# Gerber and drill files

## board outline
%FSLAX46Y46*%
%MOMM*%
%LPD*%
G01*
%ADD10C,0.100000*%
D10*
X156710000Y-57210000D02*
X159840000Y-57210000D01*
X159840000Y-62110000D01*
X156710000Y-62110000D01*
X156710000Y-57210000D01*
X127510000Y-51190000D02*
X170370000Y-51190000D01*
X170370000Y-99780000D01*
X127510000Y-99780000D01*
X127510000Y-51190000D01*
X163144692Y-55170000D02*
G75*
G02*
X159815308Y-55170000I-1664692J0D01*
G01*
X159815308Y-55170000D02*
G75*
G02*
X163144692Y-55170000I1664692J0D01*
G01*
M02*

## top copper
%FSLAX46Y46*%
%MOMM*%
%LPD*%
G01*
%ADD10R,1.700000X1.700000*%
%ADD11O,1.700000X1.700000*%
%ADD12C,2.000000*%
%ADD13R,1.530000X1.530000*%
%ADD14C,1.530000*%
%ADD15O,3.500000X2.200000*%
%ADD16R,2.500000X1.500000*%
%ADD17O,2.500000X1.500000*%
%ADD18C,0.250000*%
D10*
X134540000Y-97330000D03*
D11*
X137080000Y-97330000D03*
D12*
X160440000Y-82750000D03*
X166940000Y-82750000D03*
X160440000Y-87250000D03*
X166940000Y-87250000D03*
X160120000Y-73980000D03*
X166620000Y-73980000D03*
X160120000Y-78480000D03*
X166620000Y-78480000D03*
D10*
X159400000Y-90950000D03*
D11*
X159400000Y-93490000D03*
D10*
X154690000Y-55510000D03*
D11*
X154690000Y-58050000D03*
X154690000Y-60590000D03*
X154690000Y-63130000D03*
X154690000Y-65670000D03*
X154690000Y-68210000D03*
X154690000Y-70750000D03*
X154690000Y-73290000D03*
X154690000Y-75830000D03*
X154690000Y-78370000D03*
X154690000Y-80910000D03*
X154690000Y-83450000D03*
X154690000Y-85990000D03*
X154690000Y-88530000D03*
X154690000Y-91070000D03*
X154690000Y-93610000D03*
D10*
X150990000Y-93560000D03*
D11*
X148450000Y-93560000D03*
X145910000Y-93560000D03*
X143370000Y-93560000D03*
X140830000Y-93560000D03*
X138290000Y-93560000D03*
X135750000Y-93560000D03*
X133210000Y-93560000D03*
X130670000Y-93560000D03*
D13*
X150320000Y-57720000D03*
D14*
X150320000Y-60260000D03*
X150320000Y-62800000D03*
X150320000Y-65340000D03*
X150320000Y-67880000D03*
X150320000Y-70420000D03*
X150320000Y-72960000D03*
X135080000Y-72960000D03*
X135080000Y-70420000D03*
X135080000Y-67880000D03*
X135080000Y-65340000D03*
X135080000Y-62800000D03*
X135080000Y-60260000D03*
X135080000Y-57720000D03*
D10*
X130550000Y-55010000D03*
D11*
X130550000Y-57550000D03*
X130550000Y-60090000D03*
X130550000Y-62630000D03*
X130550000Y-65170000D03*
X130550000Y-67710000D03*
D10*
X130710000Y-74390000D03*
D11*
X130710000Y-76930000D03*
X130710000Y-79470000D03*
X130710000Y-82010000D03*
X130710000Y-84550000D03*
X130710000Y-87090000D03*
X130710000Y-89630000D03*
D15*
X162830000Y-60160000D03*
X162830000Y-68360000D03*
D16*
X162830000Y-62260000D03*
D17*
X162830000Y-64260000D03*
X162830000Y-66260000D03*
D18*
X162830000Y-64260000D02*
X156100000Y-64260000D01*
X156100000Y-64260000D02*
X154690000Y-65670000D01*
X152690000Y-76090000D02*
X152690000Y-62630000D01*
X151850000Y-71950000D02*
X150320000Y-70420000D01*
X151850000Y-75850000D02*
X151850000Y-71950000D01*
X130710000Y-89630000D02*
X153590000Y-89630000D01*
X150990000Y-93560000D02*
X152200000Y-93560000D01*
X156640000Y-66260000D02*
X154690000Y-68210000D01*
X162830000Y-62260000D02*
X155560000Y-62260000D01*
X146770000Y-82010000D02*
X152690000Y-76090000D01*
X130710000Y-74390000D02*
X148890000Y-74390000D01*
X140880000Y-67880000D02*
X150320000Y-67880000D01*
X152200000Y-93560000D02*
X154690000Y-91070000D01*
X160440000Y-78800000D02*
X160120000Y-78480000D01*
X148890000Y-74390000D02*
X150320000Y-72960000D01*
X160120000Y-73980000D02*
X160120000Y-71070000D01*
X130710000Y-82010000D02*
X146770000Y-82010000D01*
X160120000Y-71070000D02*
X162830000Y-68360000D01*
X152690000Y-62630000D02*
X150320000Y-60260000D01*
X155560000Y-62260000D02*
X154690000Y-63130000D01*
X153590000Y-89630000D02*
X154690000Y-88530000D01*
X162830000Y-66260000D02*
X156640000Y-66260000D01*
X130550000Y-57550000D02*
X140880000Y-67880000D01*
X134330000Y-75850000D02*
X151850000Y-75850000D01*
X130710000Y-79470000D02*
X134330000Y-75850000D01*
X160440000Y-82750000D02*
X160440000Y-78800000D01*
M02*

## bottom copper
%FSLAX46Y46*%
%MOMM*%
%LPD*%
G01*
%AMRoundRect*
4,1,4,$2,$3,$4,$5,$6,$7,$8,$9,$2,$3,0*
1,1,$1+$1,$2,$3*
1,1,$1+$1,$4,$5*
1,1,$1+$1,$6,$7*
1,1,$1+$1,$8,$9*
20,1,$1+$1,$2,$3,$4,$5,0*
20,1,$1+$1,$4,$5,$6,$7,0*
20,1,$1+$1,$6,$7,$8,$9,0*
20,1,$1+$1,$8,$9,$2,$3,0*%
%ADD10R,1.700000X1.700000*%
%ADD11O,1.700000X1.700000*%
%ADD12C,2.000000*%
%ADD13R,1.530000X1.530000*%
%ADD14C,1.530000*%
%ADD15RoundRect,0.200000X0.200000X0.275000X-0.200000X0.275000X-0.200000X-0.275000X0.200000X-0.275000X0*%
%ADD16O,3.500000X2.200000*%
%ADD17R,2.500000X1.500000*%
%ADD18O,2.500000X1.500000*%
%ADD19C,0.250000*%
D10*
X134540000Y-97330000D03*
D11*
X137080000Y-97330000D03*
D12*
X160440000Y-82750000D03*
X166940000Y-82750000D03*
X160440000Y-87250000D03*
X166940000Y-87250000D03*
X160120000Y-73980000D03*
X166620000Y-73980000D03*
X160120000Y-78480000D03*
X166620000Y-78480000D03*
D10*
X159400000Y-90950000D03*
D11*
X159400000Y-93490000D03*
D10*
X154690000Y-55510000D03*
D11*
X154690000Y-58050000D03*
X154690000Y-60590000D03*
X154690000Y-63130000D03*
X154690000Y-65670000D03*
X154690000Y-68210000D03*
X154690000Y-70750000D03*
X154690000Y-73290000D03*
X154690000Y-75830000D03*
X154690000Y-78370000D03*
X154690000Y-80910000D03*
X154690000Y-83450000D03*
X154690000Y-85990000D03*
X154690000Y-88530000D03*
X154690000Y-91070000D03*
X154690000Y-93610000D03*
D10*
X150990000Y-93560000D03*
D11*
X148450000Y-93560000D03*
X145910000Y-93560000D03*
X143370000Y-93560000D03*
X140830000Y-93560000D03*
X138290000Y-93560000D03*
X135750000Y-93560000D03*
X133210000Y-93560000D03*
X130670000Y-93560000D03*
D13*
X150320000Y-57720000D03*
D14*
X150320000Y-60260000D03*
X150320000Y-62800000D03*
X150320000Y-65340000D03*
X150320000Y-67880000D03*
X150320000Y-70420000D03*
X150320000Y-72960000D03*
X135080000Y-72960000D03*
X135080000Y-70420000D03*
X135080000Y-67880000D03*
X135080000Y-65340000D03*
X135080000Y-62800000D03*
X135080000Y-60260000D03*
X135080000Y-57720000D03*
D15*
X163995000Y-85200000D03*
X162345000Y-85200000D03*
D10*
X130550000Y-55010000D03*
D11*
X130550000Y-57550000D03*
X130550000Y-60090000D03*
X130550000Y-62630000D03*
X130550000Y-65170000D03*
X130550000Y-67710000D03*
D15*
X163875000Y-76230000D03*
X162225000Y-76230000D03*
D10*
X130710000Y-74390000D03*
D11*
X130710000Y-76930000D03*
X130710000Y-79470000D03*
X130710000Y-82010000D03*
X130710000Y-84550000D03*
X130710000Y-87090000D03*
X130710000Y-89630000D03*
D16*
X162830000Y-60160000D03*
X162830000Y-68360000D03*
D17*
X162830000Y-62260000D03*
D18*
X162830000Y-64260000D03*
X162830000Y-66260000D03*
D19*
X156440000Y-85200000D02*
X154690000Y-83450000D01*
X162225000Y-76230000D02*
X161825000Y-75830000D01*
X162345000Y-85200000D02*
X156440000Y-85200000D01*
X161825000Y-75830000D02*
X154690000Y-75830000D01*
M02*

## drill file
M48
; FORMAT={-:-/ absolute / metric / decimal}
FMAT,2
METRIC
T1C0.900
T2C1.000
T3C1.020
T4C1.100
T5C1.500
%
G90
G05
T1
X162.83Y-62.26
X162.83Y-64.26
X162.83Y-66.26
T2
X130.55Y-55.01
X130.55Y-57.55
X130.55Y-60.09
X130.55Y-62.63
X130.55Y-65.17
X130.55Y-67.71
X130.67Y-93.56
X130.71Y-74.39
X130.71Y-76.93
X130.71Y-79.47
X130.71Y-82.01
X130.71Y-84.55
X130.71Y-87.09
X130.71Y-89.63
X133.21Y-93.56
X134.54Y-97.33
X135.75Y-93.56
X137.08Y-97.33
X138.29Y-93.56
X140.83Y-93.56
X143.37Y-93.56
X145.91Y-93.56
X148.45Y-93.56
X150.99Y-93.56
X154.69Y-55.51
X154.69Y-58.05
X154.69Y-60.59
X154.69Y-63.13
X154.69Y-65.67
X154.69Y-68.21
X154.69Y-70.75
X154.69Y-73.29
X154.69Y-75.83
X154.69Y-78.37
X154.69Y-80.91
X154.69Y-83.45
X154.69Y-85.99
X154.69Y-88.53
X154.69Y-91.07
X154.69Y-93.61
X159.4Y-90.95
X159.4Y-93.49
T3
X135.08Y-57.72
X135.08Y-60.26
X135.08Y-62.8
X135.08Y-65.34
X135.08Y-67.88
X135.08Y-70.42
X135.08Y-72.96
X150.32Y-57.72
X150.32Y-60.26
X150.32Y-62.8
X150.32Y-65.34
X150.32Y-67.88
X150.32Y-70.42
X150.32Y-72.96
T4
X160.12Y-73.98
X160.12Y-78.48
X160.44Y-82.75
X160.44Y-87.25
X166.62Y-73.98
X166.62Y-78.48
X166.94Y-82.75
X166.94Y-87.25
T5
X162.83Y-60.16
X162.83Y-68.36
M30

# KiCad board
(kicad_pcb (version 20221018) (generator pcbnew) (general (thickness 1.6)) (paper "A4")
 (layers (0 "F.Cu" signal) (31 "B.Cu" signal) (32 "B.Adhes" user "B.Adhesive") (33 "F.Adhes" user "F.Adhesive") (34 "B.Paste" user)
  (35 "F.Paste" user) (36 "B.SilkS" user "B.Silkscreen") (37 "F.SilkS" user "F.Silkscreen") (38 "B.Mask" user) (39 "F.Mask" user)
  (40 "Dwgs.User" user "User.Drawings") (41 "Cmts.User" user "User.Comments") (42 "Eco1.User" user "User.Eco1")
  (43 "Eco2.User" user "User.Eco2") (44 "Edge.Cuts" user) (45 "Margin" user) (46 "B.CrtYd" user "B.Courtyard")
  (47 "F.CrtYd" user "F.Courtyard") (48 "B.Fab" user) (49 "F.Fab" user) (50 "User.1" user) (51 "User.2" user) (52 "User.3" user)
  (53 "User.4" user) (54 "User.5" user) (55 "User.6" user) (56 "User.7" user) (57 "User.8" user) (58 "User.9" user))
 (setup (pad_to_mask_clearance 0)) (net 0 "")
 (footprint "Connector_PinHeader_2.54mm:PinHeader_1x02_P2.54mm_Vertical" (layer "F.Cu") (at 134.54 97.33 90)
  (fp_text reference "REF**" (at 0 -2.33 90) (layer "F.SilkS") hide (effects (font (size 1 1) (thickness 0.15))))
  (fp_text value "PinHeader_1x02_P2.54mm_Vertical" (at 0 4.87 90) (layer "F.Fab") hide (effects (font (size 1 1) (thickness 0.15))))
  (pad "1" thru_hole rect (at 0 0 90) (size 1.7 1.7) (drill 1) (layers "*.Cu" "*.Mask"))
  (pad "2" thru_hole oval (at 0 2.54 90) (size 1.7 1.7) (drill 1) (layers "*.Cu" "*.Mask")))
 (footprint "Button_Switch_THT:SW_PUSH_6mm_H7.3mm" (layer "F.Cu") (at 160.44 82.75)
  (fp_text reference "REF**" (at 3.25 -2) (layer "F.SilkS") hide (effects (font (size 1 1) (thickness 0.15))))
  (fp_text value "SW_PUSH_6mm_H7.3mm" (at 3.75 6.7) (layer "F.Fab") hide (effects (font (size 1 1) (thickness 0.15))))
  (pad "1" thru_hole circle (at 0 0 90) (size 2 2) (drill 1.1) (layers "*.Cu" "*.Mask"))
  (pad "1" thru_hole circle (at 6.5 0 90) (size 2 2) (drill 1.1) (layers "*.Cu" "*.Mask"))
  (pad "2" thru_hole circle (at 0 4.5 90) (size 2 2) (drill 1.1) (layers "*.Cu" "*.Mask"))
  (pad "2" thru_hole circle (at 6.5 4.5 90) (size 2 2) (drill 1.1) (layers "*.Cu" "*.Mask")))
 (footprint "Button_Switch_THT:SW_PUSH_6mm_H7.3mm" (layer "F.Cu") (at 160.12 73.98)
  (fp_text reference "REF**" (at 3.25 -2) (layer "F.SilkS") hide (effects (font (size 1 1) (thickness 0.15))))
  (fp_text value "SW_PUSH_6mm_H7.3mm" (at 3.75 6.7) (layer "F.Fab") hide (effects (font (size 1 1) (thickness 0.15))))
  (pad "1" thru_hole circle (at 0 0 90) (size 2 2) (drill 1.1) (layers "*.Cu" "*.Mask"))
  (pad "1" thru_hole circle (at 6.5 0 90) (size 2 2) (drill 1.1) (layers "*.Cu" "*.Mask"))
  (pad "2" thru_hole circle (at 0 4.5 90) (size 2 2) (drill 1.1) (layers "*.Cu" "*.Mask"))
  (pad "2" thru_hole circle (at 6.5 4.5 90) (size 2 2) (drill 1.1) (layers "*.Cu" "*.Mask")))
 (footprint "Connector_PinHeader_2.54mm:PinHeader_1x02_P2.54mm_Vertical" (layer "F.Cu") (at 159.4 90.95)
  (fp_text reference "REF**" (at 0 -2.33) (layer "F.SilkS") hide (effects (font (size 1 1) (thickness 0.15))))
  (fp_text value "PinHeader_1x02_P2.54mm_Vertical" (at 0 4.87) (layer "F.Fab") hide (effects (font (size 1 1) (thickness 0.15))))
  (pad "1" thru_hole rect (at 0 0) (size 1.7 1.7) (drill 1) (layers "*.Cu" "*.Mask"))
  (pad "2" thru_hole oval (at 0 2.54) (size 1.7 1.7) (drill 1) (layers "*.Cu" "*.Mask")))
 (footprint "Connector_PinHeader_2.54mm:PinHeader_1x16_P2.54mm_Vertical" (layer "B.Cu") (at 154.69 55.51 180)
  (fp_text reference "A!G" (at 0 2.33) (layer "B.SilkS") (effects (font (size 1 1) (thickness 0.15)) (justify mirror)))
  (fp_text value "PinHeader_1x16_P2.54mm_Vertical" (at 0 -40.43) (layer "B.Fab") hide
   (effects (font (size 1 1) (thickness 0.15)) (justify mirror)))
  (pad "1" thru_hole rect (at 0 0 180) (size 1.7 1.7) (drill 1) (layers "*.Cu" "*.Mask"))
  (pad "2" thru_hole oval (at 0 -2.54 180) (size 1.7 1.7) (drill 1) (layers "*.Cu" "*.Mask"))
  (pad "3" thru_hole oval (at 0 -5.08 180) (size 1.7 1.7) (drill 1) (layers "*.Cu" "*.Mask"))
  (pad "4" thru_hole oval (at 0 -7.62 180) (size 1.7 1.7) (drill 1) (layers "*.Cu" "*.Mask"))
  (pad "5" thru_hole oval (at 0 -10.16 180) (size 1.7 1.7) (drill 1) (layers "*.Cu" "*.Mask"))
  (pad "6" thru_hole oval (at 0 -12.7 180) (size 1.7 1.7) (drill 1) (layers "*.Cu" "*.Mask"))
  (pad "7" thru_hole oval (at 0 -15.24 180) (size 1.7 1.7) (drill 1) (layers "*.Cu" "*.Mask"))
  (pad "8" thru_hole oval (at 0 -17.78 180) (size 1.7 1.7) (drill 1) (layers "*.Cu" "*.Mask"))
  (pad "9" thru_hole oval (at 0 -20.32 180) (size 1.7 1.7) (drill 1) (layers "*.Cu" "*.Mask"))
  (pad "10" thru_hole oval (at 0 -22.86 180) (size 1.7 1.7) (drill 1) (layers "*.Cu" "*.Mask"))
  (pad "11" thru_hole oval (at 0 -25.4 180) (size 1.7 1.7) (drill 1) (layers "*.Cu" "*.Mask"))
  (pad "12" thru_hole oval (at 0 -27.94 180) (size 1.7 1.7) (drill 1) (layers "*.Cu" "*.Mask"))
  (pad "13" thru_hole oval (at 0 -30.48 180) (size 1.7 1.7) (drill 1) (layers "*.Cu" "*.Mask"))
  (pad "14" thru_hole oval (at 0 -33.02 180) (size 1.7 1.7) (drill 1) (layers "*.Cu" "*.Mask"))
  (pad "15" thru_hole oval (at 0 -35.56 180) (size 1.7 1.7) (drill 1) (layers "*.Cu" "*.Mask"))
  (pad "16" thru_hole oval (at 0 -38.1 180) (size 1.7 1.7) (drill 1) (layers "*.Cu" "*.Mask")))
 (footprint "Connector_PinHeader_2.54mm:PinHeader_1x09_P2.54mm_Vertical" (layer "B.Cu") (at 150.99 93.56 90)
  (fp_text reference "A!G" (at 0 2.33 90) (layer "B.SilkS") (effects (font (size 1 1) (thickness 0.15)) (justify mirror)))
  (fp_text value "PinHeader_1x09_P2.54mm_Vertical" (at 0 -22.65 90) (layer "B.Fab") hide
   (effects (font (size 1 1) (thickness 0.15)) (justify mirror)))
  (pad "1" thru_hole rect (at 0 0 90) (size 1.7 1.7) (drill 1) (layers "*.Cu" "*.Mask"))
  (pad "2" thru_hole oval (at 0 -2.54 90) (size 1.7 1.7) (drill 1) (layers "*.Cu" "*.Mask"))
  (pad "3" thru_hole oval (at 0 -5.08 90) (size 1.7 1.7) (drill 1) (layers "*.Cu" "*.Mask"))
  (pad "4" thru_hole oval (at 0 -7.62 90) (size 1.7 1.7) (drill 1) (layers "*.Cu" "*.Mask"))
  (pad "5" thru_hole oval (at 0 -10.16 90) (size 1.7 1.7) (drill 1) (layers "*.Cu" "*.Mask"))
  (pad "6" thru_hole oval (at 0 -12.7 90) (size 1.7 1.7) (drill 1) (layers "*.Cu" "*.Mask"))
  (pad "7" thru_hole oval (at 0 -15.24 90) (size 1.7 1.7) (drill 1) (layers "*.Cu" "*.Mask"))
  (pad "8" thru_hole oval (at 0 -17.78 90) (size 1.7 1.7) (drill 1) (layers "*.Cu" "*.Mask"))
  (pad "9" thru_hole oval (at 0 -20.32 90) (size 1.7 1.7) (drill 1) (layers "*.Cu" "*.Mask")))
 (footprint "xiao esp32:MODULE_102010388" (layer "B.Cu") (at 142.7 65.34 180)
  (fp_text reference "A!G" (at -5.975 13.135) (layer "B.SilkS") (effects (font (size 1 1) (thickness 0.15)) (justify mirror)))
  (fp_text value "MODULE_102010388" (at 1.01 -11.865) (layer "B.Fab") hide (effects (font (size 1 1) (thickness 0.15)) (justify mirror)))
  (pad "1" thru_hole rect (at -7.62 7.62 180) (size 1.53 1.53) (drill 1.02) (layers "*.Cu" "*.Mask") (solder_mask_margin 0.102))
  (pad "2" thru_hole circle (at -7.62 5.08 180) (size 1.53 1.53) (drill 1.02) (layers "*.Cu" "*.Mask") (solder_mask_margin 0.102))
  (pad "3" thru_hole circle (at -7.62 2.54 180) (size 1.53 1.53) (drill 1.02) (layers "*.Cu" "*.Mask") (solder_mask_margin 0.102))
  (pad "4" thru_hole circle (at -7.62 0 180) (size 1.53 1.53) (drill 1.02) (layers "*.Cu" "*.Mask") (solder_mask_margin 0.102))
  (pad "5" thru_hole circle (at -7.62 -2.54 180) (size 1.53 1.53) (drill 1.02) (layers "*.Cu" "*.Mask") (solder_mask_margin 0.102))
  (pad "6" thru_hole circle (at -7.62 -5.08 180) (size 1.53 1.53) (drill 1.02) (layers "*.Cu" "*.Mask") (solder_mask_margin 0.102))
  (pad "7" thru_hole circle (at -7.62 -7.62 180) (size 1.53 1.53) (drill 1.02) (layers "*.Cu" "*.Mask") (solder_mask_margin 0.102))
  (pad "8" thru_hole circle (at 7.62 -7.62 180) (size 1.53 1.53) (drill 1.02) (layers "*.Cu" "*.Mask") (solder_mask_margin 0.102))
  (pad "9" thru_hole circle (at 7.62 -5.08 180) (size 1.53 1.53) (drill 1.02) (layers "*.Cu" "*.Mask") (solder_mask_margin 0.102))
  (pad "10" thru_hole circle (at 7.62 -2.54 180) (size 1.53 1.53) (drill 1.02) (layers "*.Cu" "*.Mask") (solder_mask_margin 0.102))
  (pad "11" thru_hole circle (at 7.62 0 180) (size 1.53 1.53) (drill 1.02) (layers "*.Cu" "*.Mask") (solder_mask_margin 0.102))
  (pad "12" thru_hole circle (at 7.62 2.54 180) (size 1.53 1.53) (drill 1.02) (layers "*.Cu" "*.Mask") (solder_mask_margin 0.102))
  (pad "13" thru_hole circle (at 7.62 5.08 180) (size 1.53 1.53) (drill 1.02) (layers "*.Cu" "*.Mask") (solder_mask_margin 0.102))
  (pad "14" thru_hole circle (at 7.62 7.62 180) (size 1.53 1.53) (drill 1.02) (layers "*.Cu" "*.Mask") (solder_mask_margin 0.102)))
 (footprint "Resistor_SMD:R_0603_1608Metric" (layer "B.Cu") (at 163.17 85.2 180)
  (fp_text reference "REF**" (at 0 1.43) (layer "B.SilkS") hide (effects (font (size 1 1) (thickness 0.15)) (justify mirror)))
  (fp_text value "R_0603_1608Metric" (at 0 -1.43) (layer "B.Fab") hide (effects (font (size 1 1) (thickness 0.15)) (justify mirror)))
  (pad "1" smd roundrect (at -0.825 0 180) (size 0.8 0.95) (layers "B.Cu" "B.Paste" "B.Mask") (roundrect_rratio 0.25))
  (pad "2" smd roundrect (at 0.825 0 180) (size 0.8 0.95) (layers "B.Cu" "B.Paste" "B.Mask") (roundrect_rratio 0.25)))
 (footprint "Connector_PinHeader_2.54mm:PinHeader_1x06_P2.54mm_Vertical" (layer "B.Cu") (at 130.55 55.01 180)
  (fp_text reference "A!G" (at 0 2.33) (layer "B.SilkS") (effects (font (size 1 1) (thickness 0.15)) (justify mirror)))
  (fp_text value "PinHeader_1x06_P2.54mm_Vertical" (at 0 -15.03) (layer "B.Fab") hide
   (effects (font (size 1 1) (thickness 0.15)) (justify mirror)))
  (pad "1" thru_hole rect (at 0 0 180) (size 1.7 1.7) (drill 1) (layers "*.Cu" "*.Mask"))
  (pad "2" thru_hole oval (at 0 -2.54 180) (size 1.7 1.7) (drill 1) (layers "*.Cu" "*.Mask"))
  (pad "3" thru_hole oval (at 0 -5.08 180) (size 1.7 1.7) (drill 1) (layers "*.Cu" "*.Mask"))
  (pad "4" thru_hole oval (at 0 -7.62 180) (size 1.7 1.7) (drill 1) (layers "*.Cu" "*.Mask"))
  (pad "5" thru_hole oval (at 0 -10.16 180) (size 1.7 1.7) (drill 1) (layers "*.Cu" "*.Mask"))
  (pad "6" thru_hole oval (at 0 -12.7 180) (size 1.7 1.7) (drill 1) (layers "*.Cu" "*.Mask")))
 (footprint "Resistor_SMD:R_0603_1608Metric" (layer "B.Cu") (at 163.05 76.23 180)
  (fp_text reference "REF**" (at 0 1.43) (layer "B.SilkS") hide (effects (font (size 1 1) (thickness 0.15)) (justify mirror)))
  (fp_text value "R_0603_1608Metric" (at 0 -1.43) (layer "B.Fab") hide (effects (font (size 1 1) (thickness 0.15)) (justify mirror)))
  (pad "1" smd roundrect (at -0.825 0 180) (size 0.8 0.95) (layers "B.Cu" "B.Paste" "B.Mask") (roundrect_rratio 0.25))
  (pad "2" smd roundrect (at 0.825 0 180) (size 0.8 0.95) (layers "B.Cu" "B.Paste" "B.Mask") (roundrect_rratio 0.25)))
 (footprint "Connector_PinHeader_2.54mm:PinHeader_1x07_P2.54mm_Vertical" (layer "B.Cu") (at 130.71 74.39 180)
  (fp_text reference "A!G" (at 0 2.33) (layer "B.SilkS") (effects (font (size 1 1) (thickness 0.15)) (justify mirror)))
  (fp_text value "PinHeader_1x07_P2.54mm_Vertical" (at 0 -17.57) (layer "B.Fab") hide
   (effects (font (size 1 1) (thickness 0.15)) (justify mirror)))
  (pad "1" thru_hole rect (at 0 0 180) (size 1.7 1.7) (drill 1) (layers "*.Cu" "*.Mask"))
  (pad "2" thru_hole oval (at 0 -2.54 180) (size 1.7 1.7) (drill 1) (layers "*.Cu" "*.Mask"))
  (pad "3" thru_hole oval (at 0 -5.08 180) (size 1.7 1.7) (drill 1) (layers "*.Cu" "*.Mask"))
  (pad "4" thru_hole oval (at 0 -7.62 180) (size 1.7 1.7) (drill 1) (layers "*.Cu" "*.Mask"))
  (pad "5" thru_hole oval (at 0 -10.16 180) (size 1.7 1.7) (drill 1) (layers "*.Cu" "*.Mask"))
  (pad "6" thru_hole oval (at 0 -12.7 180) (size 1.7 1.7) (drill 1) (layers "*.Cu" "*.Mask"))
  (pad "7" thru_hole oval (at 0 -15.24 180) (size 1.7 1.7) (drill 1) (layers "*.Cu" "*.Mask")))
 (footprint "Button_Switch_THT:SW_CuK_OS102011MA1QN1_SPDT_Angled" (layer "B.Cu") (at 162.83 62.26 -90)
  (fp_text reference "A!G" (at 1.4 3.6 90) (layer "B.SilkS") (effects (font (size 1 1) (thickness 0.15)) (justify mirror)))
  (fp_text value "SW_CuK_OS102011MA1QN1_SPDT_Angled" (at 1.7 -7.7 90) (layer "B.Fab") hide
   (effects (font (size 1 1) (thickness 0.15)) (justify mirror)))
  (pad "" thru_hole oval (at -2.1 0 270) (size 2.2 3.5) (drill 1.5) (layers "*.Cu" "*.Mask"))
  (pad "" thru_hole oval (at 6.1 0 270) (size 2.2 3.5) (drill 1.5) (layers "*.Cu" "*.Mask"))
  (pad "1" thru_hole rect (at 0 0 270) (size 1.5 2.5) (drill 0.9) (layers "*.Cu" "*.Mask"))
  (pad "2" thru_hole oval (at 2 0 270) (size 1.5 2.5) (drill 0.9) (layers "*.Cu" "*.Mask"))
  (pad "3" thru_hole oval (at 4 0 270) (size 1.5 2.5) (drill 0.9) (layers "*.Cu" "*.Mask")))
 (gr_rect (start 156.71 57.21) (end 159.84 62.11) (stroke (width 0.1) (type default)) (fill none) (layer "Edge.Cuts"))
 (gr_rect (start 127.51 51.19) (end 170.37 99.78) (stroke (width 0.1) (type default)) (fill none) (layer "Edge.Cuts"))
 (gr_circle (center 161.48 55.17) (end 163.144692 55.17) (stroke (width 0.1) (type default)) (fill none) (layer "Edge.Cuts"))
 (segment (start 162.83 64.26) (end 156.1 64.26) (width 0.25) (layer "F.Cu") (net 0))
 (segment (start 156.1 64.26) (end 154.69 65.67) (width 0.25) (layer "F.Cu") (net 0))
 (segment (start 152.69 76.09) (end 152.69 62.63) (width 0.25) (layer "F.Cu") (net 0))
 (segment (start 151.85 71.95) (end 150.32 70.42) (width 0.25) (layer "F.Cu") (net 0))
 (segment (start 151.85 75.85) (end 151.85 71.95) (width 0.25) (layer "F.Cu") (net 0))
 (segment (start 130.71 89.63) (end 153.59 89.63) (width 0.25) (layer "F.Cu") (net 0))
 (segment (start 150.99 93.56) (end 152.2 93.56) (width 0.25) (layer "F.Cu") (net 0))
 (segment (start 156.64 66.26) (end 154.69 68.21) (width 0.25) (layer "F.Cu") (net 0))
 (segment (start 162.83 62.26) (end 155.56 62.26) (width 0.25) (layer "F.Cu") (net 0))
 (segment (start 146.77 82.01) (end 152.69 76.09) (width 0.25) (layer "F.Cu") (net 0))
 (segment (start 130.71 74.39) (end 148.89 74.39) (width 0.25) (layer "F.Cu") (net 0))
 (segment (start 140.88 67.88) (end 150.32 67.88) (width 0.25) (layer "F.Cu") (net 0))
 (segment (start 152.2 93.56) (end 154.69 91.07) (width 0.25) (layer "F.Cu") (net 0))
 (segment (start 160.44 78.8) (end 160.12 78.48) (width 0.25) (layer "F.Cu") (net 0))
 (segment (start 148.89 74.39) (end 150.32 72.96) (width 0.25) (layer "F.Cu") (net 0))
 (segment (start 160.12 73.98) (end 160.12 71.07) (width 0.25) (layer "F.Cu") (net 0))
 (segment (start 130.71 82.01) (end 146.77 82.01) (width 0.25) (layer "F.Cu") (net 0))
 (segment (start 160.12 71.07) (end 162.83 68.36) (width 0.25) (layer "F.Cu") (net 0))
 (segment (start 152.69 62.63) (end 150.32 60.26) (width 0.25) (layer "F.Cu") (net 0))
 (segment (start 155.56 62.26) (end 154.69 63.13) (width 0.25) (layer "F.Cu") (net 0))
 (segment (start 153.59 89.63) (end 154.69 88.53) (width 0.25) (layer "F.Cu") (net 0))
 (segment (start 162.83 66.26) (end 156.64 66.26) (width 0.25) (layer "F.Cu") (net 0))
 (segment (start 130.55 57.55) (end 140.88 67.88) (width 0.25) (layer "F.Cu") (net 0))
 (segment (start 134.33 75.85) (end 151.85 75.85) (width 0.25) (layer "F.Cu") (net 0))
 (segment (start 130.71 79.47) (end 134.33 75.85) (width 0.25) (layer "F.Cu") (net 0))
 (segment (start 160.44 82.75) (end 160.44 78.8) (width 0.25) (layer "F.Cu") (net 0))
 (segment (start 156.44 85.2) (end 154.69 83.45) (width 0.25) (layer "B.Cu") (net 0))
 (segment (start 162.225 76.23) (end 161.825 75.83) (width 0.25) (layer "B.Cu") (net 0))
 (segment (start 162.345 85.2) (end 156.44 85.2) (width 0.25) (layer "B.Cu") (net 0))
 (segment (start 161.825 75.83) (end 154.69 75.83) (width 0.25) (layer "B.Cu") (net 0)))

